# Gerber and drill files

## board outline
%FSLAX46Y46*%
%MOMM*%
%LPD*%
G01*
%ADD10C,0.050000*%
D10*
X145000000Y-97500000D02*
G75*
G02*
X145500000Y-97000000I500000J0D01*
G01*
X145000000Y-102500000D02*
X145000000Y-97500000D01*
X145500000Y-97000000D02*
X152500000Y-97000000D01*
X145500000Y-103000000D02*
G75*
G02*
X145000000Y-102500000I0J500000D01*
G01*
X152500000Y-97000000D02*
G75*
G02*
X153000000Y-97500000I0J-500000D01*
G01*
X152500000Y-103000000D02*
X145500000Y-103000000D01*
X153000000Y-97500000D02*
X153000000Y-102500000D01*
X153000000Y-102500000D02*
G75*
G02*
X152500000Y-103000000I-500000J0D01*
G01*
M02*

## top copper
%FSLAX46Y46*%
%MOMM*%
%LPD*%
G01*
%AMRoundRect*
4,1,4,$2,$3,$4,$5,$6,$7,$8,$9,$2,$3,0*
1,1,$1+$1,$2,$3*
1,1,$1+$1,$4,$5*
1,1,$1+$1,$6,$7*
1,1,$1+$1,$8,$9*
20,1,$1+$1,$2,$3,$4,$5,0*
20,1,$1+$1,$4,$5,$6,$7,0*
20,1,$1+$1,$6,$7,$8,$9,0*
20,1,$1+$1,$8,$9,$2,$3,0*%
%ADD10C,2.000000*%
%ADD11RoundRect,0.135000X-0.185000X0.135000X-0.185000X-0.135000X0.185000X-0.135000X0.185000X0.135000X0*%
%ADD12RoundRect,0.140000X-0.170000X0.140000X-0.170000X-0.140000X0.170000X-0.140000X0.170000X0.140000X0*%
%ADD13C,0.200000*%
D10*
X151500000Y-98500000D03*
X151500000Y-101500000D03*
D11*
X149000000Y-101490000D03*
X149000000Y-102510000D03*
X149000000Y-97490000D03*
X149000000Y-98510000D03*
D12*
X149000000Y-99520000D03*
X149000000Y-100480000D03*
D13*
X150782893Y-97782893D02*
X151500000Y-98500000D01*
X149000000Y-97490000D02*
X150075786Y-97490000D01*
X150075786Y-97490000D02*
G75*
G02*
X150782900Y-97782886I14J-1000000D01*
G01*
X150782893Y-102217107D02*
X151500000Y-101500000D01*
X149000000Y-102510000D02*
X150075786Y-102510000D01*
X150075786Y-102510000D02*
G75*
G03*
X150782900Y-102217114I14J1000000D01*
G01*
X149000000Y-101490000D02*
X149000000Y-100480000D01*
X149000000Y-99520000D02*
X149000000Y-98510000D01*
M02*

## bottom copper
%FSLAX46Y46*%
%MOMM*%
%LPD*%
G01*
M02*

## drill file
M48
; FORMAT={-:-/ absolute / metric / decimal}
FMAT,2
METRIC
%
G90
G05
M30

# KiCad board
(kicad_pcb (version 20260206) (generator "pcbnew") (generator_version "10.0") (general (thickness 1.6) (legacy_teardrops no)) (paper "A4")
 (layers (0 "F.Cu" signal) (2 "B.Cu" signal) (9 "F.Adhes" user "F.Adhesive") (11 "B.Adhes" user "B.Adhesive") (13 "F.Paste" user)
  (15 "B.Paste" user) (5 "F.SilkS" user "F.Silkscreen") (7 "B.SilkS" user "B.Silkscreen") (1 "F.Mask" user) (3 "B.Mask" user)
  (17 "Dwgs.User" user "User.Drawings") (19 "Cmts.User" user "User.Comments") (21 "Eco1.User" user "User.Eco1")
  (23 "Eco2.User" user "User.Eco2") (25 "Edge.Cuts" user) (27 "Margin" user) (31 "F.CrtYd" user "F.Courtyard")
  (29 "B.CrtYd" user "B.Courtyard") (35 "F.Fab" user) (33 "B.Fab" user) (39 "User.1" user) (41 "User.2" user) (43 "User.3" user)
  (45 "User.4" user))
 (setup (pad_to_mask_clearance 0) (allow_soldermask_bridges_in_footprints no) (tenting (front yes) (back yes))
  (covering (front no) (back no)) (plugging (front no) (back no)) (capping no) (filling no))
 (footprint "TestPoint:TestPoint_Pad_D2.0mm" (layer "F.Cu") (at 151.5 98.5)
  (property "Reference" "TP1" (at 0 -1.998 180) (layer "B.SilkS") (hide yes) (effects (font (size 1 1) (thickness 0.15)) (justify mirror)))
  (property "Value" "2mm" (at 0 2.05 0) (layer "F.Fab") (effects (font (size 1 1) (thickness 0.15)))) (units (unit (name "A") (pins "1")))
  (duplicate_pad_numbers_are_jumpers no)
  (pad "1" smd circle (at 0 0) (size 2 2) (layers "F.Cu" "F.Mask") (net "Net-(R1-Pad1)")))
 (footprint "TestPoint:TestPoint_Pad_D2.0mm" (layer "F.Cu") (at 151.5 101.5)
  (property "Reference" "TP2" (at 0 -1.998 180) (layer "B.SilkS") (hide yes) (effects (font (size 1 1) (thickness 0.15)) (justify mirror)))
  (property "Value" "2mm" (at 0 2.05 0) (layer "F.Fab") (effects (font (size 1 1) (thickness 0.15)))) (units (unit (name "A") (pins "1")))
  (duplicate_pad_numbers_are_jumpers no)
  (pad "1" smd circle (at 0 0) (size 2 2) (layers "F.Cu" "F.Mask") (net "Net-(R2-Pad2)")))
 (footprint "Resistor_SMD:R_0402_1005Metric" (layer "F.Cu") (at 149 102 -90)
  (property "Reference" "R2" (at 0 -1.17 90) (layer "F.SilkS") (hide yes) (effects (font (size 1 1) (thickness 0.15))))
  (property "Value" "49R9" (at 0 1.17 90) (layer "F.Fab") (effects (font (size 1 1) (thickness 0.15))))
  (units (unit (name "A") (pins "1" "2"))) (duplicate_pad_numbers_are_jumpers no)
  (pad "1" smd roundrect (at -0.51 0 270) (size 0.54 0.64) (layers "F.Cu" "F.Mask" "F.Paste") (roundrect_rratio 0.25) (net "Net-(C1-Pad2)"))
  (pad "2" smd roundrect (at 0.51 0 270) (size 0.54 0.64) (layers "F.Cu" "F.Mask" "F.Paste") (roundrect_rratio 0.25) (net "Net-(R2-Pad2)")))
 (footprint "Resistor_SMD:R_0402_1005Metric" (layer "F.Cu") (at 149 98 -90)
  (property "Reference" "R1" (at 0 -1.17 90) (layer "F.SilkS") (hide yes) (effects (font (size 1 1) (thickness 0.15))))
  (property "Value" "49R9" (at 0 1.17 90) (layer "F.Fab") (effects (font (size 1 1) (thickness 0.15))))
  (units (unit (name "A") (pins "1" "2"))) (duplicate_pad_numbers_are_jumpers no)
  (pad "1" smd roundrect (at -0.51 0 270) (size 0.54 0.64) (layers "F.Cu" "F.Mask" "F.Paste") (roundrect_rratio 0.25) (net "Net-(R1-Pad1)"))
  (pad "2" smd roundrect (at 0.51 0 270) (size 0.54 0.64) (layers "F.Cu" "F.Mask" "F.Paste") (roundrect_rratio 0.25) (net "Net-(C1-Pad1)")))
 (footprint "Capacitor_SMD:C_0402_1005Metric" (layer "F.Cu") (at 149 100 -90)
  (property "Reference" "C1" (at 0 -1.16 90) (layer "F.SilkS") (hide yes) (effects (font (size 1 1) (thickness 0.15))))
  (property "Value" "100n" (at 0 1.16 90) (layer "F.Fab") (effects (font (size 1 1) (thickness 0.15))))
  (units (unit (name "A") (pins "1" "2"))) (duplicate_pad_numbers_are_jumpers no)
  (pad "1" smd roundrect (at -0.48 0 270) (size 0.56 0.62) (layers "F.Cu" "F.Mask" "F.Paste") (roundrect_rratio 0.25) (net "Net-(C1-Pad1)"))
  (pad "2" smd roundrect (at 0.48 0 270) (size 0.56 0.62) (layers "F.Cu" "F.Mask" "F.Paste") (roundrect_rratio 0.25) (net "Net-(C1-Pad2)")))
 (gr_arc (start 145 97.5) (mid 145.146447 97.146447) (end 145.5 97) (stroke (width 0.05) (type default)) (layer "Edge.Cuts"))
 (gr_line (start 145 102.5) (end 145 97.5) (stroke (width 0.05) (type default)) (layer "Edge.Cuts"))
 (gr_line (start 145.5 97) (end 152.5 97) (stroke (width 0.05) (type default)) (layer "Edge.Cuts"))
 (gr_arc (start 145.5 103) (mid 145.146447 102.853553) (end 145 102.5) (stroke (width 0.05) (type default)) (layer "Edge.Cuts"))
 (gr_arc (start 152.5 97) (mid 152.853553 97.146447) (end 153 97.5) (stroke (width 0.05) (type default)) (layer "Edge.Cuts"))
 (gr_line (start 152.5 103) (end 145.5 103) (stroke (width 0.05) (type default)) (layer "Edge.Cuts"))
 (gr_line (start 153 97.5) (end 153 102.5) (stroke (width 0.05) (type default)) (layer "Edge.Cuts"))
 (gr_arc (start 153 102.5) (mid 152.853553 102.853553) (end 152.5 103) (stroke (width 0.05) (type default)) (layer "Edge.Cuts"))
 (segment (start 150.782893 97.782893) (end 151.5 98.5) (width 0.2) (layer "F.Cu") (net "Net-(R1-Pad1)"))
 (segment (start 149 97.49) (end 150.075786 97.49) (width 0.2) (layer "F.Cu") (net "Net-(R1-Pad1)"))
 (arc (start 150.075786 97.49) (mid 150.458469 97.56612) (end 150.782893 97.782893) (width 0.2) (layer "F.Cu") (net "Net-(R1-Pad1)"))
 (segment (start 150.782893 102.217107) (end 151.5 101.5) (width 0.2) (layer "F.Cu") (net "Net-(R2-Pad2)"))
 (segment (start 149 102.51) (end 150.075786 102.51) (width 0.2) (layer "F.Cu") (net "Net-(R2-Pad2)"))
 (arc (start 150.075786 102.51) (mid 150.458469 102.43388) (end 150.782893 102.217107) (width 0.2) (layer "F.Cu") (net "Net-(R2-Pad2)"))
 (segment (start 149 101.49) (end 149 100.48) (width 0.2) (layer "F.Cu") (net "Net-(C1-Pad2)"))
 (segment (start 149 99.52) (end 149 98.51) (width 0.2) (layer "F.Cu") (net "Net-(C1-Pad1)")))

